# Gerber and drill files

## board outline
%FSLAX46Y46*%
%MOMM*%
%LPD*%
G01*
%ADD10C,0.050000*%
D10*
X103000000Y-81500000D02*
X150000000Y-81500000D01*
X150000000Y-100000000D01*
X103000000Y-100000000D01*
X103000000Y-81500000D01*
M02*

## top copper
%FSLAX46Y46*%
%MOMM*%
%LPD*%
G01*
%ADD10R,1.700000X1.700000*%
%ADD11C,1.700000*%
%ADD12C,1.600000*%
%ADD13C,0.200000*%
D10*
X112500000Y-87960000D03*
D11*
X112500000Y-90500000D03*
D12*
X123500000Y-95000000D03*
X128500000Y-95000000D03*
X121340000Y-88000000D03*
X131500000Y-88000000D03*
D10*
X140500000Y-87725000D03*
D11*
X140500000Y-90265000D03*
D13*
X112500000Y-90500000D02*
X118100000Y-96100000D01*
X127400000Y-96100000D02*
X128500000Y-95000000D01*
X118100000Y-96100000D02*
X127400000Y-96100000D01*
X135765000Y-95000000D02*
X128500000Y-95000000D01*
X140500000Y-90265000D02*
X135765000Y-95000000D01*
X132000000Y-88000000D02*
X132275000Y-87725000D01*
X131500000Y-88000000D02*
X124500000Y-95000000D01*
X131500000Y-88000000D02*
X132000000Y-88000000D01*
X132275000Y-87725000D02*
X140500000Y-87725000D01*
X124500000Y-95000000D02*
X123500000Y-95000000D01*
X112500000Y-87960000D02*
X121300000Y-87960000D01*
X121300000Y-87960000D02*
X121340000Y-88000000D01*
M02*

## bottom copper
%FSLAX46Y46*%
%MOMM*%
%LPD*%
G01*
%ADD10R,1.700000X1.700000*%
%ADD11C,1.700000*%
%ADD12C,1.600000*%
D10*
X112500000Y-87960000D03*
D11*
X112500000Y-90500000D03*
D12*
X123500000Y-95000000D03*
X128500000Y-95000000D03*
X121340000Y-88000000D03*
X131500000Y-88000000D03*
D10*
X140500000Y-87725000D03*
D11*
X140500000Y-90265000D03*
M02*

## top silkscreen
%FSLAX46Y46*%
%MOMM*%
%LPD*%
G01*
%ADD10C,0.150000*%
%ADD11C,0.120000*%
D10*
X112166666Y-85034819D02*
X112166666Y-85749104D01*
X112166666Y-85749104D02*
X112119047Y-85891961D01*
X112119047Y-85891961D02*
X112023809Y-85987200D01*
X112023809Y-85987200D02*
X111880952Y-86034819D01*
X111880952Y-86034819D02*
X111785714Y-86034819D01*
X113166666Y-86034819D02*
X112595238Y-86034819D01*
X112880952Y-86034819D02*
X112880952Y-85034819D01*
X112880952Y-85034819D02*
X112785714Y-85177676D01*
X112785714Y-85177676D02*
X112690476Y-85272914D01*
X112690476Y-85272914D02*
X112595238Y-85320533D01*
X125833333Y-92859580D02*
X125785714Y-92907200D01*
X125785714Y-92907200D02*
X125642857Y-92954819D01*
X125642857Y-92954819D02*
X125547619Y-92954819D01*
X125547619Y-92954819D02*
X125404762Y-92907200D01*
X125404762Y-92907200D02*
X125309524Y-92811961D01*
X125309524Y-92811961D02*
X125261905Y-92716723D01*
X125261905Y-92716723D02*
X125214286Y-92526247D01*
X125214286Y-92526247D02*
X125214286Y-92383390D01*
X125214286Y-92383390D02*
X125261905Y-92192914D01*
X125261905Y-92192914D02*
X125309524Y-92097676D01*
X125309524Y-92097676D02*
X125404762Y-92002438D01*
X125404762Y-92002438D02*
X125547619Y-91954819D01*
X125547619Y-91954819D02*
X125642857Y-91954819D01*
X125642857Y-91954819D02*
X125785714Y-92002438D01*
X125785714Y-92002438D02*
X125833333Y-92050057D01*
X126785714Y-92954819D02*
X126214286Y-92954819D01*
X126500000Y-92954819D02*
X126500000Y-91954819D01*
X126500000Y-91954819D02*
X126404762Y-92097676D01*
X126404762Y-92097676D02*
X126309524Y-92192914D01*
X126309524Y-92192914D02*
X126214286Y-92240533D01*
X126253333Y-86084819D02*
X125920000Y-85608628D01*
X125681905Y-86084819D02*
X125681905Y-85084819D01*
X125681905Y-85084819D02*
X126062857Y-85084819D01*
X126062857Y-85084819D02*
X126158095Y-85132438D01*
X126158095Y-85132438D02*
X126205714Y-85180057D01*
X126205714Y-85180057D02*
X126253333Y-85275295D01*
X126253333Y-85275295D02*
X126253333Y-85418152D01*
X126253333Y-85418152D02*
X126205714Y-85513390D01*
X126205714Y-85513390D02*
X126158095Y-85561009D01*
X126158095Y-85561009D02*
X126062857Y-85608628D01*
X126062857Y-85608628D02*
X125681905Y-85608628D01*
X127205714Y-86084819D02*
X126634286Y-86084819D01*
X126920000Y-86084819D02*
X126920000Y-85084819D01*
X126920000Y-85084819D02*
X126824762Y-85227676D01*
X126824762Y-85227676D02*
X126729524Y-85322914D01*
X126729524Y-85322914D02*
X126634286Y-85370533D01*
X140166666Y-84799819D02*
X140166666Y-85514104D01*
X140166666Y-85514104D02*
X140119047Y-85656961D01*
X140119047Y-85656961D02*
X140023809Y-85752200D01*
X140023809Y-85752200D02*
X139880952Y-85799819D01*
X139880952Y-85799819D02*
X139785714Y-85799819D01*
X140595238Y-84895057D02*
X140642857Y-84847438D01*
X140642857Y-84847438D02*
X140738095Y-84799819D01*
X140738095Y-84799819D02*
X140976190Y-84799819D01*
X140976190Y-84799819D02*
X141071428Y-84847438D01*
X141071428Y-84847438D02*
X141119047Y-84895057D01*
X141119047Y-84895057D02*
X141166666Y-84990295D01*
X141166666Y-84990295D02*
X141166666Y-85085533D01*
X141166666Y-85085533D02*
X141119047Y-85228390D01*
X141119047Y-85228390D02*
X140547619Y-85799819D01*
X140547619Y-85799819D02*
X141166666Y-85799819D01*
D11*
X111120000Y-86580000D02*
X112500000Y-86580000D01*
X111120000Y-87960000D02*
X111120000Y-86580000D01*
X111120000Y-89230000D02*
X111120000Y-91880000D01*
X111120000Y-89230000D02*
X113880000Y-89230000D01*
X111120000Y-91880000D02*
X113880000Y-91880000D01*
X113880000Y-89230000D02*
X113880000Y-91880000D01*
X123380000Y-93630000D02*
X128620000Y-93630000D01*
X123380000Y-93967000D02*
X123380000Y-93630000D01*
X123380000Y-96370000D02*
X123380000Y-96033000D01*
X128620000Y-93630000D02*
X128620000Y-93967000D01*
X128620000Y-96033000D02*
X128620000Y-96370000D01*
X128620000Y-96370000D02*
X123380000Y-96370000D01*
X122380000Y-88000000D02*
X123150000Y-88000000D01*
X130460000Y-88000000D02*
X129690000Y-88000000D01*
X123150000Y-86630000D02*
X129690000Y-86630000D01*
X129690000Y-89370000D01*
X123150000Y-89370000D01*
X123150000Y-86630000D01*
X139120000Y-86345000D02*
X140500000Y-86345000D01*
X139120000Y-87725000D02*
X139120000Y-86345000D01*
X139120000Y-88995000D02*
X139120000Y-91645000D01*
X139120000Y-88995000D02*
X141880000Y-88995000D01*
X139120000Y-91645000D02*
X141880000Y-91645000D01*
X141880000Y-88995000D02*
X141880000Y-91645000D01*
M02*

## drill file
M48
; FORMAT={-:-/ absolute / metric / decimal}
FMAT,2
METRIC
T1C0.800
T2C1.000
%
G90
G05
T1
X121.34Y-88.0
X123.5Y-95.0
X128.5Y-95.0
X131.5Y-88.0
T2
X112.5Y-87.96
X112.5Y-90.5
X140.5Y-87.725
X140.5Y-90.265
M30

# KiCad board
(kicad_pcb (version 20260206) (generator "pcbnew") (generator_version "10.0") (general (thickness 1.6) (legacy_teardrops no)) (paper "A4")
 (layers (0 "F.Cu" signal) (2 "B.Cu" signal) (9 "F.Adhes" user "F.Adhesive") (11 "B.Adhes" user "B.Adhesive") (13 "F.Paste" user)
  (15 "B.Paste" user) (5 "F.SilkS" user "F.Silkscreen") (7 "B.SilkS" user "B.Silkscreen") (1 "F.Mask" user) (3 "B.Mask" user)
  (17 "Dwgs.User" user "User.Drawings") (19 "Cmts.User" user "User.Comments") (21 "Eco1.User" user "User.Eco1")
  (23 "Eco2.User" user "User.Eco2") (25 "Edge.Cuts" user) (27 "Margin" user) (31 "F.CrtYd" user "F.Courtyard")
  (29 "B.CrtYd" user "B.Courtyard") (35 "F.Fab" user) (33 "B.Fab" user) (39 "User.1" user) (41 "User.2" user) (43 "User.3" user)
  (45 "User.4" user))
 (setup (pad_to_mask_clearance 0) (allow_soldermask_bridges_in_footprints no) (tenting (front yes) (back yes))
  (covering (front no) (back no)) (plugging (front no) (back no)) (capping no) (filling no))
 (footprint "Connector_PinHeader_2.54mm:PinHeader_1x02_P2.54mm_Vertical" (layer "F.Cu") (at 112.5 87.96)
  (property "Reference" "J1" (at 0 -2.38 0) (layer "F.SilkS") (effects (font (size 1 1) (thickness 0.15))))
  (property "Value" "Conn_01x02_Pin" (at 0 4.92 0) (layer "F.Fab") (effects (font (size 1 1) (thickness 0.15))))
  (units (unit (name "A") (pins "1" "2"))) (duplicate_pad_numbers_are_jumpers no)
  (fp_line (start -1.38 -1.38) (end 0 -1.38) (stroke (width 0.12) (type solid)) (layer "F.SilkS"))
  (fp_line (start -1.38 0) (end -1.38 -1.38) (stroke (width 0.12) (type solid)) (layer "F.SilkS"))
  (fp_line (start -1.38 1.27) (end -1.38 3.92) (stroke (width 0.12) (type solid)) (layer "F.SilkS"))
  (fp_line (start -1.38 1.27) (end 1.38 1.27) (stroke (width 0.12) (type solid)) (layer "F.SilkS"))
  (fp_line (start -1.38 3.92) (end 1.38 3.92) (stroke (width 0.12) (type solid)) (layer "F.SilkS"))
  (fp_line (start 1.38 1.27) (end 1.38 3.92) (stroke (width 0.12) (type solid)) (layer "F.SilkS"))
  (pad "1" thru_hole rect (at 0 0) (size 1.7 1.7) (drill 1) (layers "*.Cu" "*.Mask") (remove_unused_layers no) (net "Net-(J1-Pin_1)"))
  (pad "2" thru_hole circle (at 0 2.54) (size 1.7 1.7) (drill 1) (layers "*.Cu" "*.Mask") (remove_unused_layers no) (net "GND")))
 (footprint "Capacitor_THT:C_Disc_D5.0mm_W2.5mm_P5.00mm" (layer "F.Cu") (at 123.5 95)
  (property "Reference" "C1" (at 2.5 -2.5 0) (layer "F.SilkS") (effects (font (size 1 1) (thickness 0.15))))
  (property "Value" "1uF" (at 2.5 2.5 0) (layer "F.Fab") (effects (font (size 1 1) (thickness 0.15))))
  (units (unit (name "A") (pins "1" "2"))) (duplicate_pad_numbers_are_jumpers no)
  (fp_line (start -0.12 -1.37) (end 5.12 -1.37) (stroke (width 0.12) (type solid)) (layer "F.SilkS"))
  (fp_line (start -0.12 -1.033) (end -0.12 -1.37) (stroke (width 0.12) (type solid)) (layer "F.SilkS"))
  (fp_line (start -0.12 1.37) (end -0.12 1.033) (stroke (width 0.12) (type solid)) (layer "F.SilkS"))
  (fp_line (start 5.12 -1.37) (end 5.12 -1.033) (stroke (width 0.12) (type solid)) (layer "F.SilkS"))
  (fp_line (start 5.12 1.033) (end 5.12 1.37) (stroke (width 0.12) (type solid)) (layer "F.SilkS"))
  (fp_line (start 5.12 1.37) (end -0.12 1.37) (stroke (width 0.12) (type solid)) (layer "F.SilkS"))
  (pad "1" thru_hole circle (at 0 0) (size 1.6 1.6) (drill 0.8) (layers "*.Cu" "*.Mask") (remove_unused_layers no) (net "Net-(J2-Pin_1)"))
  (pad "2" thru_hole circle (at 5 0) (size 1.6 1.6) (drill 0.8) (layers "*.Cu" "*.Mask") (remove_unused_layers no) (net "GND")))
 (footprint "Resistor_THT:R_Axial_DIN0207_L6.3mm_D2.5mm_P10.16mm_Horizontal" (layer "F.Cu") (at 121.34 88)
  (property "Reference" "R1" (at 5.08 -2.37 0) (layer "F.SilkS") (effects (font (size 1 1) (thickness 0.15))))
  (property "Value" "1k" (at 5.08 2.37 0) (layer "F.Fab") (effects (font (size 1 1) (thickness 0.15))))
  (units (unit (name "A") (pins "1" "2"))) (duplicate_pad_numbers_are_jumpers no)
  (fp_line (start 1.04 0) (end 1.81 0) (stroke (width 0.12) (type solid)) (layer "F.SilkS"))
  (fp_line (start 9.12 0) (end 8.35 0) (stroke (width 0.12) (type solid)) (layer "F.SilkS"))
  (fp_rect (start 1.81 -1.37) (end 8.35 1.37) (stroke (width 0.12) (type solid)) (fill no) (layer "F.SilkS"))
  (pad "1" thru_hole circle (at 0 0) (size 1.6 1.6) (drill 0.8) (layers "*.Cu" "*.Mask") (remove_unused_layers no) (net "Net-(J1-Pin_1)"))
  (pad "2" thru_hole circle (at 10.16 0) (size 1.6 1.6) (drill 0.8) (layers "*.Cu" "*.Mask") (remove_unused_layers no)
   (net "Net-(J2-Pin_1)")))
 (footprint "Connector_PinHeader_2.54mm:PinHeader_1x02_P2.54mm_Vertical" (layer "F.Cu") (at 140.5 87.725)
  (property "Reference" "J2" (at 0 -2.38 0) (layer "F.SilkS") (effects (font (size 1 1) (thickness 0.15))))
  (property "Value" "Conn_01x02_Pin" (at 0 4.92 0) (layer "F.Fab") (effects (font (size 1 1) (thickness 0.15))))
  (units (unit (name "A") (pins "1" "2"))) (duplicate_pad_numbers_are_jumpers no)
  (fp_line (start -1.38 -1.38) (end 0 -1.38) (stroke (width 0.12) (type solid)) (layer "F.SilkS"))
  (fp_line (start -1.38 0) (end -1.38 -1.38) (stroke (width 0.12) (type solid)) (layer "F.SilkS"))
  (fp_line (start -1.38 1.27) (end -1.38 3.92) (stroke (width 0.12) (type solid)) (layer "F.SilkS"))
  (fp_line (start -1.38 1.27) (end 1.38 1.27) (stroke (width 0.12) (type solid)) (layer "F.SilkS"))
  (fp_line (start -1.38 3.92) (end 1.38 3.92) (stroke (width 0.12) (type solid)) (layer "F.SilkS"))
  (fp_line (start 1.38 1.27) (end 1.38 3.92) (stroke (width 0.12) (type solid)) (layer "F.SilkS"))
  (pad "1" thru_hole rect (at 0 0) (size 1.7 1.7) (drill 1) (layers "*.Cu" "*.Mask") (remove_unused_layers no) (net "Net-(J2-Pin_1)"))
  (pad "2" thru_hole circle (at 0 2.54) (size 1.7 1.7) (drill 1) (layers "*.Cu" "*.Mask") (remove_unused_layers no) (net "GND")))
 (gr_rect (start 103 81.5) (end 150 100) (stroke (width 0.05) (type default)) (fill no) (layer "Edge.Cuts"))
 (segment (start 112.5 90.5) (end 118.1 96.1) (width 0.2) (layer "F.Cu") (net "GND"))
 (segment (start 127.4 96.1) (end 128.5 95) (width 0.2) (layer "F.Cu") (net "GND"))
 (segment (start 118.1 96.1) (end 127.4 96.1) (width 0.2) (layer "F.Cu") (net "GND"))
 (segment (start 135.765 95) (end 128.5 95) (width 0.2) (layer "F.Cu") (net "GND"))
 (segment (start 140.5 90.265) (end 135.765 95) (width 0.2) (layer "F.Cu") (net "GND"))
 (segment (start 132 88) (end 132.275 87.725) (width 0.2) (layer "F.Cu") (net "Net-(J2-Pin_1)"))
 (segment (start 131.5 88) (end 124.5 95) (width 0.2) (layer "F.Cu") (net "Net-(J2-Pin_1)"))
 (segment (start 131.5 88) (end 132 88) (width 0.2) (layer "F.Cu") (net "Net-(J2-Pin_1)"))
 (segment (start 132.275 87.725) (end 140.5 87.725) (width 0.2) (layer "F.Cu") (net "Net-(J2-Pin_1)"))
 (segment (start 124.5 95) (end 123.5 95) (width 0.2) (layer "F.Cu") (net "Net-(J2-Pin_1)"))
 (segment (start 112.5 87.96) (end 121.3 87.96) (width 0.2) (layer "F.Cu") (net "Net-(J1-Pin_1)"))
 (segment (start 121.3 87.96) (end 121.34 88) (width 0.2) (layer "F.Cu") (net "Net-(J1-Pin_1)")))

